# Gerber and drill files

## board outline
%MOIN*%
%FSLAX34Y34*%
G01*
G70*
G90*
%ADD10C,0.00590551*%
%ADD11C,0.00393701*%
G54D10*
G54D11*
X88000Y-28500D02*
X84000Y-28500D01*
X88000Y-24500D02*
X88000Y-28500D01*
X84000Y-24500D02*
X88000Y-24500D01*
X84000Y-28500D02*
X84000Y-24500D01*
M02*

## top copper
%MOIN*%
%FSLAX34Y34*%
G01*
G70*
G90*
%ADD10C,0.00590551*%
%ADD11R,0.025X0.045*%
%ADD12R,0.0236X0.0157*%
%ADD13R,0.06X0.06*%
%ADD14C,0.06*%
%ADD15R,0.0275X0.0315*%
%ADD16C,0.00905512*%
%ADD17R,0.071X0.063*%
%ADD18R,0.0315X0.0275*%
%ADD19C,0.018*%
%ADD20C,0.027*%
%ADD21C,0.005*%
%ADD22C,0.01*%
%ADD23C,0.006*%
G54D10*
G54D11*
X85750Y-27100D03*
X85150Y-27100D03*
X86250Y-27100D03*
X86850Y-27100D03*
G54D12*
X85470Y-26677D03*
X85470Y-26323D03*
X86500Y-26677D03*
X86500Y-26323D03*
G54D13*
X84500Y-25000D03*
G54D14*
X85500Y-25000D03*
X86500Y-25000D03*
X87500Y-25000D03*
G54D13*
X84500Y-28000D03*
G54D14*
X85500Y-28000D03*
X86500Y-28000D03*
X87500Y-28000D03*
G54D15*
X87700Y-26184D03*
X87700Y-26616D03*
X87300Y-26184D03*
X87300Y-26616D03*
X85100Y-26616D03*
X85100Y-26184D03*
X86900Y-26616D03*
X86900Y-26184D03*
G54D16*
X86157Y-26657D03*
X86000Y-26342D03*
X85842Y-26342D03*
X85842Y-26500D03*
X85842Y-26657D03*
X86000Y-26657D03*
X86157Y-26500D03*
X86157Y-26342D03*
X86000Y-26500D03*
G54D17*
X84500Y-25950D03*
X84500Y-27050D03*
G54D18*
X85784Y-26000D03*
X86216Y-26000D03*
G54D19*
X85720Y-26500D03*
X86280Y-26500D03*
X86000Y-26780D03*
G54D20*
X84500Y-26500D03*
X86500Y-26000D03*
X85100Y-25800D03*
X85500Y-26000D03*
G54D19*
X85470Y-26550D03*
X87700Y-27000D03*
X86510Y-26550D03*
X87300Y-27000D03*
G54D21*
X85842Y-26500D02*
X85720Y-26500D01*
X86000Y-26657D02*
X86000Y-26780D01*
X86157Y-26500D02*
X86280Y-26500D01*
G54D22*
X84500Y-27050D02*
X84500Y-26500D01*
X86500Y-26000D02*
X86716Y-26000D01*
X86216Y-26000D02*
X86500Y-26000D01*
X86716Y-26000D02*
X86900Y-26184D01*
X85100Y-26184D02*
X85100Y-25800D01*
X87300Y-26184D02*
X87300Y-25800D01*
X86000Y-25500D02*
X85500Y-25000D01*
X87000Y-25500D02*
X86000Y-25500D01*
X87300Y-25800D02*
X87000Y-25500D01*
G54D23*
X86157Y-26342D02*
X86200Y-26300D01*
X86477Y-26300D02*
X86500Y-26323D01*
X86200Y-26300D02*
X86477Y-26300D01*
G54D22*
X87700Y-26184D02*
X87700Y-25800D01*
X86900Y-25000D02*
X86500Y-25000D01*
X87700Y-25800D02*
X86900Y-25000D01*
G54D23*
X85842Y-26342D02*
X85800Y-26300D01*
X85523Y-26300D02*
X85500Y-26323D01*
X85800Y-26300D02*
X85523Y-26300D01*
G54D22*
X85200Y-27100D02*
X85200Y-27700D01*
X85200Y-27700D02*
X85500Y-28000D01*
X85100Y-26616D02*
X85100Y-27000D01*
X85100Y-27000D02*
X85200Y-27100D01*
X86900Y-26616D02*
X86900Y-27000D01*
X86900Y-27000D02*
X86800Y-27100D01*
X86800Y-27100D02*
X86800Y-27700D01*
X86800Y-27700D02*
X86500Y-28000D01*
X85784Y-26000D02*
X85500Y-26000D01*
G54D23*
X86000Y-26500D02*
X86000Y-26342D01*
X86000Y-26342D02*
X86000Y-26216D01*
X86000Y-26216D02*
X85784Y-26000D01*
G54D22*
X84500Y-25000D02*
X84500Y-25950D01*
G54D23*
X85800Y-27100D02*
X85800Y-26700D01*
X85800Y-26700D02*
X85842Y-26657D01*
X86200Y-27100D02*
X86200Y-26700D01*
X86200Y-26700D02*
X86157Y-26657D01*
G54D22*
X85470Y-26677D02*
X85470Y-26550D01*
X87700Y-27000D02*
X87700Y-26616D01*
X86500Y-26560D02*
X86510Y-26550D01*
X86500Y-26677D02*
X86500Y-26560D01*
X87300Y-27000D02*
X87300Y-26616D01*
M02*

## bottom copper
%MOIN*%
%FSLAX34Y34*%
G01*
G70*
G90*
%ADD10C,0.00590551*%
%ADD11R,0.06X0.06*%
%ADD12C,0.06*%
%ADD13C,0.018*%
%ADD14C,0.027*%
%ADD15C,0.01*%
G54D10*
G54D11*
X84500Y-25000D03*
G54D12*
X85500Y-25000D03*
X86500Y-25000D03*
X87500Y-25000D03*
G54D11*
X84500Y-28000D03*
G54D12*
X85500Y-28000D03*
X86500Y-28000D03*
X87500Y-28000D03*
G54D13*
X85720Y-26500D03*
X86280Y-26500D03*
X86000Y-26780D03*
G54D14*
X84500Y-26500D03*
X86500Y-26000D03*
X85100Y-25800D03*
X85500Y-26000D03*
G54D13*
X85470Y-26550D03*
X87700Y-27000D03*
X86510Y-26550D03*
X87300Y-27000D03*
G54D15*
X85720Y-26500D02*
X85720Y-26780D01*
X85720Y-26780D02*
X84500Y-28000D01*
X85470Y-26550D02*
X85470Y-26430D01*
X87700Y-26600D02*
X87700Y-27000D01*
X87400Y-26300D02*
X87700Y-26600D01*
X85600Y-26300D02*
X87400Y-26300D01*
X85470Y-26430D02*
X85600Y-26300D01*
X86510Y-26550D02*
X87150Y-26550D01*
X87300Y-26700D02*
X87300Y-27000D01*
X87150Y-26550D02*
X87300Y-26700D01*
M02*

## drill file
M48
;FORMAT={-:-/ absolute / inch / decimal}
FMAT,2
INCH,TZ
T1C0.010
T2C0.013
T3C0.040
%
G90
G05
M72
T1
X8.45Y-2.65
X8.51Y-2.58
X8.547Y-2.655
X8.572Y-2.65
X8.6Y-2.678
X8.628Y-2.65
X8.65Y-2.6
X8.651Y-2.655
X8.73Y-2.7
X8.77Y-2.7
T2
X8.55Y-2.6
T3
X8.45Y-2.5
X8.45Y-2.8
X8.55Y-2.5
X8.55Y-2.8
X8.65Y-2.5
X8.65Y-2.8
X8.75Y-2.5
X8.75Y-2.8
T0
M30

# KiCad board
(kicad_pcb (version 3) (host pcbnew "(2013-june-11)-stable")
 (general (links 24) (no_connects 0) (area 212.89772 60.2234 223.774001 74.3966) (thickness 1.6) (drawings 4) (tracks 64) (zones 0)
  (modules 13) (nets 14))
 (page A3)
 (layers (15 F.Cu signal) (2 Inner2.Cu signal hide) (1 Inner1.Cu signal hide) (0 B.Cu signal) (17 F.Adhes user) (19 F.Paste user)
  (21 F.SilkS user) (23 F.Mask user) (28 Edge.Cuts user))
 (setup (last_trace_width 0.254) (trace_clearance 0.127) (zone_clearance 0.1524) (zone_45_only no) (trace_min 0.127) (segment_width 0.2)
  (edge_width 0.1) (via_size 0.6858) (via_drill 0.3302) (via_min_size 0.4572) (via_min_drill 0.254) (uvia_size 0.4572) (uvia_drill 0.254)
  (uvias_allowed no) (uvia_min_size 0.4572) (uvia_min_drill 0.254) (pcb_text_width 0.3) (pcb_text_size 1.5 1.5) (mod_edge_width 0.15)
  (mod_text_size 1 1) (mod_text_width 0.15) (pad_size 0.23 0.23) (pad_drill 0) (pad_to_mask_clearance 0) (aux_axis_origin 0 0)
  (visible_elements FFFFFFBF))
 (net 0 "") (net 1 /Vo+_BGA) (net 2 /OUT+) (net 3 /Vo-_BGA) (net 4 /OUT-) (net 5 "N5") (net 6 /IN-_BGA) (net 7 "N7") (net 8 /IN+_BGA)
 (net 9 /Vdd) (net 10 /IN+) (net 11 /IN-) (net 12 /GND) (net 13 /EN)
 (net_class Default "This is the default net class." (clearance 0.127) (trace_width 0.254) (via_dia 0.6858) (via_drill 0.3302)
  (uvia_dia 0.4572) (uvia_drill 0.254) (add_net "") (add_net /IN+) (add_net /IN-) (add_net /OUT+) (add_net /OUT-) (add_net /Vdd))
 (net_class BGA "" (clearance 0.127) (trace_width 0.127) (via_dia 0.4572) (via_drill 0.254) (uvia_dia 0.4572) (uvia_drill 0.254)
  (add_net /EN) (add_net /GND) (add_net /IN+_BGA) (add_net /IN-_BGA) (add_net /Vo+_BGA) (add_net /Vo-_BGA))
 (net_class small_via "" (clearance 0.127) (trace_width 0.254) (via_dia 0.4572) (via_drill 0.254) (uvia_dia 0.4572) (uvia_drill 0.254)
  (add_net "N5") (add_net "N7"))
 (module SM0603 (layer F.Cu) (at 217.043 68.834 180)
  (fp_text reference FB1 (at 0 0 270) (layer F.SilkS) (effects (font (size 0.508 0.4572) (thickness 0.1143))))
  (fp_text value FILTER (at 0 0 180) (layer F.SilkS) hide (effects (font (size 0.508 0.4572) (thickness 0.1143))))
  (pad 1 smd rect (at -0.762 0 180) (size 0.635 1.143) (layers F.Cu F.Paste F.Mask) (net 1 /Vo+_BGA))
  (pad 2 smd rect (at 0.762 0 180) (size 0.635 1.143) (layers F.Cu F.Paste F.Mask) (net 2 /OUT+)))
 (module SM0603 (layer F.Cu) (at 219.837 68.834)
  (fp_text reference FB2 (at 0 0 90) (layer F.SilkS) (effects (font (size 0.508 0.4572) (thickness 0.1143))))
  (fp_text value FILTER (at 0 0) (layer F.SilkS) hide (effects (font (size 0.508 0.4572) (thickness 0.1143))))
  (pad 1 smd rect (at -0.762 0) (size 0.635 1.143) (layers F.Cu F.Paste F.Mask) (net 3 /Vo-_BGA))
  (pad 2 smd rect (at 0.762 0) (size 0.635 1.143) (layers F.Cu F.Paste F.Mask) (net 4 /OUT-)))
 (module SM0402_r (layer F.Cu) (at 217.0938 67.31 90) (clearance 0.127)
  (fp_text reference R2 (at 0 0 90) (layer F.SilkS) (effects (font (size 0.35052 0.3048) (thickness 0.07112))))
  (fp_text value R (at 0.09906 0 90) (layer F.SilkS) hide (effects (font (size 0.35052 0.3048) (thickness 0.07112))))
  (pad 1 smd rect (at -0.44958 0 90) (size 0.39878 0.59944) (layers F.Cu F.Paste F.Mask) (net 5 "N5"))
  (pad 2 smd rect (at 0.44958 0 90) (size 0.39878 0.59944) (layers F.Cu F.Paste F.Mask) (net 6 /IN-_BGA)))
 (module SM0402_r (layer F.Cu) (at 219.71 67.31 90)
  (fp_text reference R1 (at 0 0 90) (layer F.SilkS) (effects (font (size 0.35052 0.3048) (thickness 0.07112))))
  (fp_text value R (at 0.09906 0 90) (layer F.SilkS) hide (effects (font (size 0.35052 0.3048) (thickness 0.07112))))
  (pad 1 smd rect (at -0.44958 0 90) (size 0.39878 0.59944) (layers F.Cu F.Paste F.Mask) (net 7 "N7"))
  (pad 2 smd rect (at 0.44958 0 90) (size 0.39878 0.59944) (layers F.Cu F.Paste F.Mask) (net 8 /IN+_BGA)))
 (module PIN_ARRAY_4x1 (layer B.Cu) (at 218.44 63.5)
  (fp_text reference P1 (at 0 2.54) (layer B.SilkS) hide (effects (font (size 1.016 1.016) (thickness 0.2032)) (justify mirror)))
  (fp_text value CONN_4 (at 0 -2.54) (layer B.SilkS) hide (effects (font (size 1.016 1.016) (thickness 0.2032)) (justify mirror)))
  (pad 1 thru_hole rect (at -3.81 0) (size 1.524 1.524) (drill 1.016) (layers *.Cu *.Mask) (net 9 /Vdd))
  (pad 2 thru_hole circle (at -1.27 0) (size 1.524 1.524) (drill 1.016) (layers *.Cu *.Mask) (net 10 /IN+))
  (pad 3 thru_hole circle (at 1.27 0) (size 1.524 1.524) (drill 1.016) (layers *.Cu *.Mask) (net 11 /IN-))
  (pad 4 thru_hole circle (at 3.81 0) (size 1.524 1.524) (drill 1.016) (layers *.Cu *.Mask) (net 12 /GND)))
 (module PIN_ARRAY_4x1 (layer B.Cu) (at 218.44 71.12)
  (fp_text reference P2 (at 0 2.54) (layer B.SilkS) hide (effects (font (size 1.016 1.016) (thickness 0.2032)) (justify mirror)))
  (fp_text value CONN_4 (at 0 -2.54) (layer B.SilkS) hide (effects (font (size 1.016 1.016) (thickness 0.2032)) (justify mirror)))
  (pad 1 thru_hole rect (at -3.81 0) (size 1.524 1.524) (drill 1.016) (layers *.Cu *.Mask) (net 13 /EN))
  (pad 2 thru_hole circle (at -1.27 0) (size 1.524 1.524) (drill 1.016) (layers *.Cu *.Mask) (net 2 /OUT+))
  (pad 3 thru_hole circle (at 1.27 0) (size 1.524 1.524) (drill 1.016) (layers *.Cu *.Mask) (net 4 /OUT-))
  (pad 4 thru_hole circle (at 3.81 0) (size 1.524 1.524) (drill 1.016) (layers *.Cu *.Mask) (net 12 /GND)))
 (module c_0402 (layer F.Cu) (at 222.758 67.056 90)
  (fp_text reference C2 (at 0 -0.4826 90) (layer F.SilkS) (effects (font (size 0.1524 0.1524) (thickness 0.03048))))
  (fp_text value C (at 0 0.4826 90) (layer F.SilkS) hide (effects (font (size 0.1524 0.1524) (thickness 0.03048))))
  (pad 1 smd rect (at 0.54864 0 90) (size 0.8001 0.6985) (layers F.Cu F.Paste F.Mask) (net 11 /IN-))
  (pad 2 smd rect (at -0.54864 0 90) (size 0.8001 0.6985) (layers F.Cu F.Paste F.Mask) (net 5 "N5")))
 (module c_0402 (layer F.Cu) (at 221.742 67.056 90)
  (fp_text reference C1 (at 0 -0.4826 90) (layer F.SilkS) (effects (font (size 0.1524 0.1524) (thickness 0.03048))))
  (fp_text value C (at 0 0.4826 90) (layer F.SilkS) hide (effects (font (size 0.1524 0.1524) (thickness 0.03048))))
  (pad 1 smd rect (at 0.54864 0 90) (size 0.8001 0.6985) (layers F.Cu F.Paste F.Mask) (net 10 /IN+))
  (pad 2 smd rect (at -0.54864 0 90) (size 0.8001 0.6985) (layers F.Cu F.Paste F.Mask) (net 7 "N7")))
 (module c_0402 (layer F.Cu) (at 216.154 67.056 270)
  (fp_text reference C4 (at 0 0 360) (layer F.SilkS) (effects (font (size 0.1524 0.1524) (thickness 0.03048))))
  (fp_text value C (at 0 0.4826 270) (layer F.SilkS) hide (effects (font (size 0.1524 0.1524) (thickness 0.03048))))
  (pad 1 smd rect (at 0.54864 0 270) (size 0.8001 0.6985) (layers F.Cu F.Paste F.Mask) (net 2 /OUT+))
  (pad 2 smd rect (at -0.54864 0 270) (size 0.8001 0.6985) (layers F.Cu F.Paste F.Mask) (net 12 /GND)))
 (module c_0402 (layer F.Cu) (at 220.726 67.056 270)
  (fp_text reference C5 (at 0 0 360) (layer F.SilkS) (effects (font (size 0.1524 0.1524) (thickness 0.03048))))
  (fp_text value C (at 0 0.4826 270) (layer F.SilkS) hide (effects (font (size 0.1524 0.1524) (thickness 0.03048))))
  (pad 1 smd rect (at 0.54864 0 270) (size 0.8001 0.6985) (layers F.Cu F.Paste F.Mask) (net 4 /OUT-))
  (pad 2 smd rect (at -0.54864 0 270) (size 0.8001 0.6985) (layers F.Cu F.Paste F.Mask) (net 12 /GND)))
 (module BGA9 (layer F.Cu) (at 218.44 67.31 270) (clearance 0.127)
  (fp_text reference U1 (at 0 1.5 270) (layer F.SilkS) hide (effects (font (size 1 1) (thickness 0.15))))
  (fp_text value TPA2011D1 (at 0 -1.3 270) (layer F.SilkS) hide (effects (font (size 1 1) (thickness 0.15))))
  (pad A3 smd circle (at 0.4 -0.4 270) (size 0.23 0.23) (layers F.Cu F.Paste F.Mask) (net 3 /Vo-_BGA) (solder_mask_margin 0.04)
   (clearance 0.16))
  (pad B1 smd circle (at -0.4 0 270) (size 0.23 0.23) (layers F.Cu F.Paste F.Mask) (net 9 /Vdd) (solder_mask_margin 0.04) (clearance 0.16))
  (pad C1 smd circle (at -0.4 0.4 270) (size 0.23 0.23) (layers F.Cu F.Paste F.Mask) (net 6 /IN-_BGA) (solder_mask_margin 0.04)
   (clearance 0.16))
  (pad C2 smd circle (at 0 0.4 270) (size 0.23 0.23) (layers F.Cu F.Paste F.Mask) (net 13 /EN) (solder_mask_margin 0.04) (clearance 0.16))
  (pad C3 smd circle (at 0.4 0.4 270) (size 0.23 0.23) (layers F.Cu F.Paste F.Mask) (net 1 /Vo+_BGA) (solder_mask_margin 0.04)
   (clearance 0.16))
  (pad B3 smd circle (at 0.4 0 270) (size 0.23 0.23) (layers F.Cu F.Paste F.Mask) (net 12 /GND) (solder_mask_margin 0.04) (clearance 0.16))
  (pad A2 smd circle (at 0 -0.4 270) (size 0.23 0.23) (layers F.Cu F.Paste F.Mask) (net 12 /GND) (solder_mask_margin 0.04) (clearance 0.16))
  (pad A1 smd circle (at -0.4 -0.4 270) (size 0.23 0.23) (layers F.Cu F.Paste F.Mask) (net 8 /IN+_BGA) (solder_mask_margin 0.04)
   (clearance 0.16))
  (pad B2 smd circle (at 0 0 270) (size 0.23 0.23) (layers F.Cu F.Paste F.Mask) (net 9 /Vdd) (solder_mask_margin 0.04) (clearance 0.16)))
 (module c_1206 (layer F.Cu) (at 214.63 67.31 90)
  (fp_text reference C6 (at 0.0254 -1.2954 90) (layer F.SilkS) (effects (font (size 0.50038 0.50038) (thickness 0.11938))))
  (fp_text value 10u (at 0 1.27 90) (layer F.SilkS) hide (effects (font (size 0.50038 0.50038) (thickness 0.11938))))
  (pad 1 smd rect (at 1.397 0 90) (size 1.6002 1.8034) (layers F.Cu F.Paste F.Mask) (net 9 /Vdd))
  (pad 2 smd rect (at -1.397 0 90) (size 1.6002 1.8034) (layers F.Cu F.Paste F.Mask) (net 12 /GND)))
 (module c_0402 (layer F.Cu) (at 218.44 66.04 180)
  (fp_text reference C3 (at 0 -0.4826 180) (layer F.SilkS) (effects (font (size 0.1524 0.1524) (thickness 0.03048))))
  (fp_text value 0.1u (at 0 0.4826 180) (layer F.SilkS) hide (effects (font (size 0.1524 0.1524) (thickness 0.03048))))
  (pad 1 smd rect (at 0.54864 0 180) (size 0.8001 0.6985) (layers F.Cu F.Paste F.Mask) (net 9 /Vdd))
  (pad 2 smd rect (at -0.54864 0 180) (size 0.8001 0.6985) (layers F.Cu F.Paste F.Mask) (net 12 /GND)))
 (gr_line (start 223.52 72.39) (end 213.36 72.39) (angle 90) (layer Edge.Cuts) (width 0.1))
 (gr_line (start 223.52 62.23) (end 223.52 72.39) (angle 90) (layer Edge.Cuts) (width 0.1))
 (gr_line (start 213.36 62.23) (end 223.52 62.23) (angle 90) (layer Edge.Cuts) (width 0.1))
 (gr_line (start 213.36 72.39) (end 213.36 62.23) (angle 90) (layer Edge.Cuts) (width 0.1))
 (via (at 217.7288 67.31) (size 0.4572) (layers F.Cu B.Cu) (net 13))
 (segment (start 218.04 67.31) (end 217.7288 67.31) (width 0.127) (layer F.Cu) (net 13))
 (segment (start 217.7288 67.31) (end 217.7288 68.0212) (width 0.254) (layer B.Cu) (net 13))
 (segment (start 217.7288 68.0212) (end 214.63 71.12) (width 0.254) (layer B.Cu) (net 13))
 (via (at 219.1512 67.31) (size 0.4572) (layers F.Cu B.Cu) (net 12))
 (via (at 218.44 68.0212) (size 0.4572) (layers F.Cu B.Cu) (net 12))
 (segment (start 218.44 67.71) (end 218.44 68.0212) (width 0.127) (layer F.Cu) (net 12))
 (segment (start 218.84 67.31) (end 219.1512 67.31) (width 0.127) (layer F.Cu) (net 12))
 (segment (start 214.63 68.707) (end 214.63 67.31) (width 0.254) (layer F.Cu) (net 12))
 (via (at 214.63 67.31) (size 0.6858) (layers F.Cu B.Cu) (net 12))
 (segment (start 219.71 66.04) (end 220.25864 66.04) (width 0.254) (layer F.Cu) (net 12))
 (via (at 219.71 66.04) (size 0.6858) (layers F.Cu B.Cu) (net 12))
 (segment (start 218.98864 66.04) (end 219.71 66.04) (width 0.254) (layer F.Cu) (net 12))
 (segment (start 220.25864 66.04) (end 220.726 66.50736) (width 0.254) (layer F.Cu) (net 12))
 (segment (start 216.154 66.50736) (end 216.154 65.532) (width 0.254) (layer F.Cu) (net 12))
 (via (at 216.154 65.532) (size 0.6858) (layers F.Cu B.Cu) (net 12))
 (segment (start 221.742 66.50736) (end 221.742 65.532) (width 0.254) (layer F.Cu) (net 10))
 (segment (start 218.44 64.77) (end 217.17 63.5) (width 0.254) (layer F.Cu) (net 10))
 (segment (start 220.98 64.77) (end 218.44 64.77) (width 0.254) (layer F.Cu) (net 10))
 (segment (start 221.742 65.532) (end 220.98 64.77) (width 0.254) (layer F.Cu) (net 10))
 (segment (start 218.84 66.91) (end 218.948 66.802) (width 0.1524) (layer F.Cu) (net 8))
 (segment (start 219.65158 66.802) (end 219.71 66.86042) (width 0.1524) (layer F.Cu) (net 8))
 (segment (start 218.948 66.802) (end 219.65158 66.802) (width 0.1524) (layer F.Cu) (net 8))
 (segment (start 222.758 66.50736) (end 222.758 65.532) (width 0.254) (layer F.Cu) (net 11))
 (segment (start 220.726 63.5) (end 219.71 63.5) (width 0.254) (layer F.Cu) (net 11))
 (segment (start 222.758 65.532) (end 220.726 63.5) (width 0.254) (layer F.Cu) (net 11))
 (segment (start 218.04 66.91) (end 217.932 66.802) (width 0.1524) (layer F.Cu) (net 6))
 (segment (start 217.22842 66.802) (end 217.17 66.86042) (width 0.1524) (layer F.Cu) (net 6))
 (segment (start 217.932 66.802) (end 217.22842 66.802) (width 0.1524) (layer F.Cu) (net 6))
 (segment (start 216.408 68.834) (end 216.408 70.358) (width 0.254) (layer F.Cu) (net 2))
 (segment (start 216.408 70.358) (end 217.17 71.12) (width 0.254) (layer F.Cu) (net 2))
 (segment (start 216.154 67.60464) (end 216.154 68.58) (width 0.254) (layer F.Cu) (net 2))
 (segment (start 216.154 68.58) (end 216.408 68.834) (width 0.254) (layer F.Cu) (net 2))
 (segment (start 220.726 67.60464) (end 220.726 68.58) (width 0.254) (layer F.Cu) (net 4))
 (segment (start 220.726 68.58) (end 220.472 68.834) (width 0.254) (layer F.Cu) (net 4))
 (segment (start 220.472 68.834) (end 220.472 70.358) (width 0.254) (layer F.Cu) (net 4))
 (segment (start 220.472 70.358) (end 219.71 71.12) (width 0.254) (layer F.Cu) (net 4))
 (segment (start 217.89136 66.04) (end 217.17 66.04) (width 0.254) (layer F.Cu) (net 9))
 (via (at 217.17 66.04) (size 0.6858) (layers F.Cu B.Cu) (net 9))
 (segment (start 218.44 67.31) (end 218.44 66.91) (width 0.1524) (layer F.Cu) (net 9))
 (segment (start 218.44 66.91) (end 218.44 66.58864) (width 0.1524) (layer F.Cu) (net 9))
 (segment (start 218.44 66.58864) (end 217.89136 66.04) (width 0.1524) (layer F.Cu) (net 9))
 (segment (start 214.63 63.5) (end 214.63 65.913) (width 0.254) (layer F.Cu) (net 9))
 (segment (start 217.932 68.834) (end 217.932 67.818) (width 0.1524) (layer F.Cu) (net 1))
 (segment (start 217.932 67.818) (end 218.04 67.71) (width 0.1524) (layer F.Cu) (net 1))
 (segment (start 218.948 68.834) (end 218.948 67.818) (width 0.1524) (layer F.Cu) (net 3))
 (segment (start 218.948 67.818) (end 218.84 67.71) (width 0.1524) (layer F.Cu) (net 3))
 (segment (start 217.0938 67.437) (end 217.0938 67.1322) (width 0.254) (layer B.Cu) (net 5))
 (via (at 217.0938 67.437) (size 0.4572) (layers F.Cu B.Cu) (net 5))
 (segment (start 217.0938 67.75958) (end 217.0938 67.437) (width 0.254) (layer F.Cu) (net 5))
 (segment (start 222.758 68.58) (end 222.758 67.60464) (width 0.254) (layer F.Cu) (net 5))
 (via (at 222.758 68.58) (size 0.4572) (layers F.Cu B.Cu) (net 5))
 (segment (start 222.758 67.564) (end 222.758 68.58) (width 0.254) (layer B.Cu) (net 5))
 (segment (start 221.996 66.802) (end 222.758 67.564) (width 0.254) (layer B.Cu) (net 5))
 (segment (start 217.424 66.802) (end 221.996 66.802) (width 0.254) (layer B.Cu) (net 5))
 (segment (start 217.0938 67.1322) (end 217.424 66.802) (width 0.254) (layer B.Cu) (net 5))
 (segment (start 219.7354 67.437) (end 221.361 67.437) (width 0.254) (layer B.Cu) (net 7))
 (segment (start 219.71 67.4624) (end 219.7354 67.437) (width 0.254) (layer F.Cu) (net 7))
 (via (at 219.7354 67.437) (size 0.4572) (layers F.Cu B.Cu) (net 7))
 (segment (start 219.71 67.75958) (end 219.71 67.4624) (width 0.254) (layer F.Cu) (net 7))
 (segment (start 221.742 68.58) (end 221.742 67.60464) (width 0.254) (layer F.Cu) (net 7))
 (via (at 221.742 68.58) (size 0.4572) (layers F.Cu B.Cu) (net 7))
 (segment (start 221.742 67.818) (end 221.742 68.58) (width 0.254) (layer B.Cu) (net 7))
 (segment (start 221.361 67.437) (end 221.742 67.818) (width 0.254) (layer B.Cu) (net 7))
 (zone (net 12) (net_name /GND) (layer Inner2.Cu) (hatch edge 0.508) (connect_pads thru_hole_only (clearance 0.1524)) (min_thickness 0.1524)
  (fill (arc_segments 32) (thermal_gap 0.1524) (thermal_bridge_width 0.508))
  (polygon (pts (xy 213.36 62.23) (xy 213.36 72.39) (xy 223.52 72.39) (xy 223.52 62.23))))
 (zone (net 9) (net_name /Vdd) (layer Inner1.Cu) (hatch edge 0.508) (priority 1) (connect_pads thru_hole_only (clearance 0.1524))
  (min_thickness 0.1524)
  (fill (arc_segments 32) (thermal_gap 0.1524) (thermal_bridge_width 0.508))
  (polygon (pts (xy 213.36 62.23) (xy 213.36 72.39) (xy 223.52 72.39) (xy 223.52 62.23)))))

